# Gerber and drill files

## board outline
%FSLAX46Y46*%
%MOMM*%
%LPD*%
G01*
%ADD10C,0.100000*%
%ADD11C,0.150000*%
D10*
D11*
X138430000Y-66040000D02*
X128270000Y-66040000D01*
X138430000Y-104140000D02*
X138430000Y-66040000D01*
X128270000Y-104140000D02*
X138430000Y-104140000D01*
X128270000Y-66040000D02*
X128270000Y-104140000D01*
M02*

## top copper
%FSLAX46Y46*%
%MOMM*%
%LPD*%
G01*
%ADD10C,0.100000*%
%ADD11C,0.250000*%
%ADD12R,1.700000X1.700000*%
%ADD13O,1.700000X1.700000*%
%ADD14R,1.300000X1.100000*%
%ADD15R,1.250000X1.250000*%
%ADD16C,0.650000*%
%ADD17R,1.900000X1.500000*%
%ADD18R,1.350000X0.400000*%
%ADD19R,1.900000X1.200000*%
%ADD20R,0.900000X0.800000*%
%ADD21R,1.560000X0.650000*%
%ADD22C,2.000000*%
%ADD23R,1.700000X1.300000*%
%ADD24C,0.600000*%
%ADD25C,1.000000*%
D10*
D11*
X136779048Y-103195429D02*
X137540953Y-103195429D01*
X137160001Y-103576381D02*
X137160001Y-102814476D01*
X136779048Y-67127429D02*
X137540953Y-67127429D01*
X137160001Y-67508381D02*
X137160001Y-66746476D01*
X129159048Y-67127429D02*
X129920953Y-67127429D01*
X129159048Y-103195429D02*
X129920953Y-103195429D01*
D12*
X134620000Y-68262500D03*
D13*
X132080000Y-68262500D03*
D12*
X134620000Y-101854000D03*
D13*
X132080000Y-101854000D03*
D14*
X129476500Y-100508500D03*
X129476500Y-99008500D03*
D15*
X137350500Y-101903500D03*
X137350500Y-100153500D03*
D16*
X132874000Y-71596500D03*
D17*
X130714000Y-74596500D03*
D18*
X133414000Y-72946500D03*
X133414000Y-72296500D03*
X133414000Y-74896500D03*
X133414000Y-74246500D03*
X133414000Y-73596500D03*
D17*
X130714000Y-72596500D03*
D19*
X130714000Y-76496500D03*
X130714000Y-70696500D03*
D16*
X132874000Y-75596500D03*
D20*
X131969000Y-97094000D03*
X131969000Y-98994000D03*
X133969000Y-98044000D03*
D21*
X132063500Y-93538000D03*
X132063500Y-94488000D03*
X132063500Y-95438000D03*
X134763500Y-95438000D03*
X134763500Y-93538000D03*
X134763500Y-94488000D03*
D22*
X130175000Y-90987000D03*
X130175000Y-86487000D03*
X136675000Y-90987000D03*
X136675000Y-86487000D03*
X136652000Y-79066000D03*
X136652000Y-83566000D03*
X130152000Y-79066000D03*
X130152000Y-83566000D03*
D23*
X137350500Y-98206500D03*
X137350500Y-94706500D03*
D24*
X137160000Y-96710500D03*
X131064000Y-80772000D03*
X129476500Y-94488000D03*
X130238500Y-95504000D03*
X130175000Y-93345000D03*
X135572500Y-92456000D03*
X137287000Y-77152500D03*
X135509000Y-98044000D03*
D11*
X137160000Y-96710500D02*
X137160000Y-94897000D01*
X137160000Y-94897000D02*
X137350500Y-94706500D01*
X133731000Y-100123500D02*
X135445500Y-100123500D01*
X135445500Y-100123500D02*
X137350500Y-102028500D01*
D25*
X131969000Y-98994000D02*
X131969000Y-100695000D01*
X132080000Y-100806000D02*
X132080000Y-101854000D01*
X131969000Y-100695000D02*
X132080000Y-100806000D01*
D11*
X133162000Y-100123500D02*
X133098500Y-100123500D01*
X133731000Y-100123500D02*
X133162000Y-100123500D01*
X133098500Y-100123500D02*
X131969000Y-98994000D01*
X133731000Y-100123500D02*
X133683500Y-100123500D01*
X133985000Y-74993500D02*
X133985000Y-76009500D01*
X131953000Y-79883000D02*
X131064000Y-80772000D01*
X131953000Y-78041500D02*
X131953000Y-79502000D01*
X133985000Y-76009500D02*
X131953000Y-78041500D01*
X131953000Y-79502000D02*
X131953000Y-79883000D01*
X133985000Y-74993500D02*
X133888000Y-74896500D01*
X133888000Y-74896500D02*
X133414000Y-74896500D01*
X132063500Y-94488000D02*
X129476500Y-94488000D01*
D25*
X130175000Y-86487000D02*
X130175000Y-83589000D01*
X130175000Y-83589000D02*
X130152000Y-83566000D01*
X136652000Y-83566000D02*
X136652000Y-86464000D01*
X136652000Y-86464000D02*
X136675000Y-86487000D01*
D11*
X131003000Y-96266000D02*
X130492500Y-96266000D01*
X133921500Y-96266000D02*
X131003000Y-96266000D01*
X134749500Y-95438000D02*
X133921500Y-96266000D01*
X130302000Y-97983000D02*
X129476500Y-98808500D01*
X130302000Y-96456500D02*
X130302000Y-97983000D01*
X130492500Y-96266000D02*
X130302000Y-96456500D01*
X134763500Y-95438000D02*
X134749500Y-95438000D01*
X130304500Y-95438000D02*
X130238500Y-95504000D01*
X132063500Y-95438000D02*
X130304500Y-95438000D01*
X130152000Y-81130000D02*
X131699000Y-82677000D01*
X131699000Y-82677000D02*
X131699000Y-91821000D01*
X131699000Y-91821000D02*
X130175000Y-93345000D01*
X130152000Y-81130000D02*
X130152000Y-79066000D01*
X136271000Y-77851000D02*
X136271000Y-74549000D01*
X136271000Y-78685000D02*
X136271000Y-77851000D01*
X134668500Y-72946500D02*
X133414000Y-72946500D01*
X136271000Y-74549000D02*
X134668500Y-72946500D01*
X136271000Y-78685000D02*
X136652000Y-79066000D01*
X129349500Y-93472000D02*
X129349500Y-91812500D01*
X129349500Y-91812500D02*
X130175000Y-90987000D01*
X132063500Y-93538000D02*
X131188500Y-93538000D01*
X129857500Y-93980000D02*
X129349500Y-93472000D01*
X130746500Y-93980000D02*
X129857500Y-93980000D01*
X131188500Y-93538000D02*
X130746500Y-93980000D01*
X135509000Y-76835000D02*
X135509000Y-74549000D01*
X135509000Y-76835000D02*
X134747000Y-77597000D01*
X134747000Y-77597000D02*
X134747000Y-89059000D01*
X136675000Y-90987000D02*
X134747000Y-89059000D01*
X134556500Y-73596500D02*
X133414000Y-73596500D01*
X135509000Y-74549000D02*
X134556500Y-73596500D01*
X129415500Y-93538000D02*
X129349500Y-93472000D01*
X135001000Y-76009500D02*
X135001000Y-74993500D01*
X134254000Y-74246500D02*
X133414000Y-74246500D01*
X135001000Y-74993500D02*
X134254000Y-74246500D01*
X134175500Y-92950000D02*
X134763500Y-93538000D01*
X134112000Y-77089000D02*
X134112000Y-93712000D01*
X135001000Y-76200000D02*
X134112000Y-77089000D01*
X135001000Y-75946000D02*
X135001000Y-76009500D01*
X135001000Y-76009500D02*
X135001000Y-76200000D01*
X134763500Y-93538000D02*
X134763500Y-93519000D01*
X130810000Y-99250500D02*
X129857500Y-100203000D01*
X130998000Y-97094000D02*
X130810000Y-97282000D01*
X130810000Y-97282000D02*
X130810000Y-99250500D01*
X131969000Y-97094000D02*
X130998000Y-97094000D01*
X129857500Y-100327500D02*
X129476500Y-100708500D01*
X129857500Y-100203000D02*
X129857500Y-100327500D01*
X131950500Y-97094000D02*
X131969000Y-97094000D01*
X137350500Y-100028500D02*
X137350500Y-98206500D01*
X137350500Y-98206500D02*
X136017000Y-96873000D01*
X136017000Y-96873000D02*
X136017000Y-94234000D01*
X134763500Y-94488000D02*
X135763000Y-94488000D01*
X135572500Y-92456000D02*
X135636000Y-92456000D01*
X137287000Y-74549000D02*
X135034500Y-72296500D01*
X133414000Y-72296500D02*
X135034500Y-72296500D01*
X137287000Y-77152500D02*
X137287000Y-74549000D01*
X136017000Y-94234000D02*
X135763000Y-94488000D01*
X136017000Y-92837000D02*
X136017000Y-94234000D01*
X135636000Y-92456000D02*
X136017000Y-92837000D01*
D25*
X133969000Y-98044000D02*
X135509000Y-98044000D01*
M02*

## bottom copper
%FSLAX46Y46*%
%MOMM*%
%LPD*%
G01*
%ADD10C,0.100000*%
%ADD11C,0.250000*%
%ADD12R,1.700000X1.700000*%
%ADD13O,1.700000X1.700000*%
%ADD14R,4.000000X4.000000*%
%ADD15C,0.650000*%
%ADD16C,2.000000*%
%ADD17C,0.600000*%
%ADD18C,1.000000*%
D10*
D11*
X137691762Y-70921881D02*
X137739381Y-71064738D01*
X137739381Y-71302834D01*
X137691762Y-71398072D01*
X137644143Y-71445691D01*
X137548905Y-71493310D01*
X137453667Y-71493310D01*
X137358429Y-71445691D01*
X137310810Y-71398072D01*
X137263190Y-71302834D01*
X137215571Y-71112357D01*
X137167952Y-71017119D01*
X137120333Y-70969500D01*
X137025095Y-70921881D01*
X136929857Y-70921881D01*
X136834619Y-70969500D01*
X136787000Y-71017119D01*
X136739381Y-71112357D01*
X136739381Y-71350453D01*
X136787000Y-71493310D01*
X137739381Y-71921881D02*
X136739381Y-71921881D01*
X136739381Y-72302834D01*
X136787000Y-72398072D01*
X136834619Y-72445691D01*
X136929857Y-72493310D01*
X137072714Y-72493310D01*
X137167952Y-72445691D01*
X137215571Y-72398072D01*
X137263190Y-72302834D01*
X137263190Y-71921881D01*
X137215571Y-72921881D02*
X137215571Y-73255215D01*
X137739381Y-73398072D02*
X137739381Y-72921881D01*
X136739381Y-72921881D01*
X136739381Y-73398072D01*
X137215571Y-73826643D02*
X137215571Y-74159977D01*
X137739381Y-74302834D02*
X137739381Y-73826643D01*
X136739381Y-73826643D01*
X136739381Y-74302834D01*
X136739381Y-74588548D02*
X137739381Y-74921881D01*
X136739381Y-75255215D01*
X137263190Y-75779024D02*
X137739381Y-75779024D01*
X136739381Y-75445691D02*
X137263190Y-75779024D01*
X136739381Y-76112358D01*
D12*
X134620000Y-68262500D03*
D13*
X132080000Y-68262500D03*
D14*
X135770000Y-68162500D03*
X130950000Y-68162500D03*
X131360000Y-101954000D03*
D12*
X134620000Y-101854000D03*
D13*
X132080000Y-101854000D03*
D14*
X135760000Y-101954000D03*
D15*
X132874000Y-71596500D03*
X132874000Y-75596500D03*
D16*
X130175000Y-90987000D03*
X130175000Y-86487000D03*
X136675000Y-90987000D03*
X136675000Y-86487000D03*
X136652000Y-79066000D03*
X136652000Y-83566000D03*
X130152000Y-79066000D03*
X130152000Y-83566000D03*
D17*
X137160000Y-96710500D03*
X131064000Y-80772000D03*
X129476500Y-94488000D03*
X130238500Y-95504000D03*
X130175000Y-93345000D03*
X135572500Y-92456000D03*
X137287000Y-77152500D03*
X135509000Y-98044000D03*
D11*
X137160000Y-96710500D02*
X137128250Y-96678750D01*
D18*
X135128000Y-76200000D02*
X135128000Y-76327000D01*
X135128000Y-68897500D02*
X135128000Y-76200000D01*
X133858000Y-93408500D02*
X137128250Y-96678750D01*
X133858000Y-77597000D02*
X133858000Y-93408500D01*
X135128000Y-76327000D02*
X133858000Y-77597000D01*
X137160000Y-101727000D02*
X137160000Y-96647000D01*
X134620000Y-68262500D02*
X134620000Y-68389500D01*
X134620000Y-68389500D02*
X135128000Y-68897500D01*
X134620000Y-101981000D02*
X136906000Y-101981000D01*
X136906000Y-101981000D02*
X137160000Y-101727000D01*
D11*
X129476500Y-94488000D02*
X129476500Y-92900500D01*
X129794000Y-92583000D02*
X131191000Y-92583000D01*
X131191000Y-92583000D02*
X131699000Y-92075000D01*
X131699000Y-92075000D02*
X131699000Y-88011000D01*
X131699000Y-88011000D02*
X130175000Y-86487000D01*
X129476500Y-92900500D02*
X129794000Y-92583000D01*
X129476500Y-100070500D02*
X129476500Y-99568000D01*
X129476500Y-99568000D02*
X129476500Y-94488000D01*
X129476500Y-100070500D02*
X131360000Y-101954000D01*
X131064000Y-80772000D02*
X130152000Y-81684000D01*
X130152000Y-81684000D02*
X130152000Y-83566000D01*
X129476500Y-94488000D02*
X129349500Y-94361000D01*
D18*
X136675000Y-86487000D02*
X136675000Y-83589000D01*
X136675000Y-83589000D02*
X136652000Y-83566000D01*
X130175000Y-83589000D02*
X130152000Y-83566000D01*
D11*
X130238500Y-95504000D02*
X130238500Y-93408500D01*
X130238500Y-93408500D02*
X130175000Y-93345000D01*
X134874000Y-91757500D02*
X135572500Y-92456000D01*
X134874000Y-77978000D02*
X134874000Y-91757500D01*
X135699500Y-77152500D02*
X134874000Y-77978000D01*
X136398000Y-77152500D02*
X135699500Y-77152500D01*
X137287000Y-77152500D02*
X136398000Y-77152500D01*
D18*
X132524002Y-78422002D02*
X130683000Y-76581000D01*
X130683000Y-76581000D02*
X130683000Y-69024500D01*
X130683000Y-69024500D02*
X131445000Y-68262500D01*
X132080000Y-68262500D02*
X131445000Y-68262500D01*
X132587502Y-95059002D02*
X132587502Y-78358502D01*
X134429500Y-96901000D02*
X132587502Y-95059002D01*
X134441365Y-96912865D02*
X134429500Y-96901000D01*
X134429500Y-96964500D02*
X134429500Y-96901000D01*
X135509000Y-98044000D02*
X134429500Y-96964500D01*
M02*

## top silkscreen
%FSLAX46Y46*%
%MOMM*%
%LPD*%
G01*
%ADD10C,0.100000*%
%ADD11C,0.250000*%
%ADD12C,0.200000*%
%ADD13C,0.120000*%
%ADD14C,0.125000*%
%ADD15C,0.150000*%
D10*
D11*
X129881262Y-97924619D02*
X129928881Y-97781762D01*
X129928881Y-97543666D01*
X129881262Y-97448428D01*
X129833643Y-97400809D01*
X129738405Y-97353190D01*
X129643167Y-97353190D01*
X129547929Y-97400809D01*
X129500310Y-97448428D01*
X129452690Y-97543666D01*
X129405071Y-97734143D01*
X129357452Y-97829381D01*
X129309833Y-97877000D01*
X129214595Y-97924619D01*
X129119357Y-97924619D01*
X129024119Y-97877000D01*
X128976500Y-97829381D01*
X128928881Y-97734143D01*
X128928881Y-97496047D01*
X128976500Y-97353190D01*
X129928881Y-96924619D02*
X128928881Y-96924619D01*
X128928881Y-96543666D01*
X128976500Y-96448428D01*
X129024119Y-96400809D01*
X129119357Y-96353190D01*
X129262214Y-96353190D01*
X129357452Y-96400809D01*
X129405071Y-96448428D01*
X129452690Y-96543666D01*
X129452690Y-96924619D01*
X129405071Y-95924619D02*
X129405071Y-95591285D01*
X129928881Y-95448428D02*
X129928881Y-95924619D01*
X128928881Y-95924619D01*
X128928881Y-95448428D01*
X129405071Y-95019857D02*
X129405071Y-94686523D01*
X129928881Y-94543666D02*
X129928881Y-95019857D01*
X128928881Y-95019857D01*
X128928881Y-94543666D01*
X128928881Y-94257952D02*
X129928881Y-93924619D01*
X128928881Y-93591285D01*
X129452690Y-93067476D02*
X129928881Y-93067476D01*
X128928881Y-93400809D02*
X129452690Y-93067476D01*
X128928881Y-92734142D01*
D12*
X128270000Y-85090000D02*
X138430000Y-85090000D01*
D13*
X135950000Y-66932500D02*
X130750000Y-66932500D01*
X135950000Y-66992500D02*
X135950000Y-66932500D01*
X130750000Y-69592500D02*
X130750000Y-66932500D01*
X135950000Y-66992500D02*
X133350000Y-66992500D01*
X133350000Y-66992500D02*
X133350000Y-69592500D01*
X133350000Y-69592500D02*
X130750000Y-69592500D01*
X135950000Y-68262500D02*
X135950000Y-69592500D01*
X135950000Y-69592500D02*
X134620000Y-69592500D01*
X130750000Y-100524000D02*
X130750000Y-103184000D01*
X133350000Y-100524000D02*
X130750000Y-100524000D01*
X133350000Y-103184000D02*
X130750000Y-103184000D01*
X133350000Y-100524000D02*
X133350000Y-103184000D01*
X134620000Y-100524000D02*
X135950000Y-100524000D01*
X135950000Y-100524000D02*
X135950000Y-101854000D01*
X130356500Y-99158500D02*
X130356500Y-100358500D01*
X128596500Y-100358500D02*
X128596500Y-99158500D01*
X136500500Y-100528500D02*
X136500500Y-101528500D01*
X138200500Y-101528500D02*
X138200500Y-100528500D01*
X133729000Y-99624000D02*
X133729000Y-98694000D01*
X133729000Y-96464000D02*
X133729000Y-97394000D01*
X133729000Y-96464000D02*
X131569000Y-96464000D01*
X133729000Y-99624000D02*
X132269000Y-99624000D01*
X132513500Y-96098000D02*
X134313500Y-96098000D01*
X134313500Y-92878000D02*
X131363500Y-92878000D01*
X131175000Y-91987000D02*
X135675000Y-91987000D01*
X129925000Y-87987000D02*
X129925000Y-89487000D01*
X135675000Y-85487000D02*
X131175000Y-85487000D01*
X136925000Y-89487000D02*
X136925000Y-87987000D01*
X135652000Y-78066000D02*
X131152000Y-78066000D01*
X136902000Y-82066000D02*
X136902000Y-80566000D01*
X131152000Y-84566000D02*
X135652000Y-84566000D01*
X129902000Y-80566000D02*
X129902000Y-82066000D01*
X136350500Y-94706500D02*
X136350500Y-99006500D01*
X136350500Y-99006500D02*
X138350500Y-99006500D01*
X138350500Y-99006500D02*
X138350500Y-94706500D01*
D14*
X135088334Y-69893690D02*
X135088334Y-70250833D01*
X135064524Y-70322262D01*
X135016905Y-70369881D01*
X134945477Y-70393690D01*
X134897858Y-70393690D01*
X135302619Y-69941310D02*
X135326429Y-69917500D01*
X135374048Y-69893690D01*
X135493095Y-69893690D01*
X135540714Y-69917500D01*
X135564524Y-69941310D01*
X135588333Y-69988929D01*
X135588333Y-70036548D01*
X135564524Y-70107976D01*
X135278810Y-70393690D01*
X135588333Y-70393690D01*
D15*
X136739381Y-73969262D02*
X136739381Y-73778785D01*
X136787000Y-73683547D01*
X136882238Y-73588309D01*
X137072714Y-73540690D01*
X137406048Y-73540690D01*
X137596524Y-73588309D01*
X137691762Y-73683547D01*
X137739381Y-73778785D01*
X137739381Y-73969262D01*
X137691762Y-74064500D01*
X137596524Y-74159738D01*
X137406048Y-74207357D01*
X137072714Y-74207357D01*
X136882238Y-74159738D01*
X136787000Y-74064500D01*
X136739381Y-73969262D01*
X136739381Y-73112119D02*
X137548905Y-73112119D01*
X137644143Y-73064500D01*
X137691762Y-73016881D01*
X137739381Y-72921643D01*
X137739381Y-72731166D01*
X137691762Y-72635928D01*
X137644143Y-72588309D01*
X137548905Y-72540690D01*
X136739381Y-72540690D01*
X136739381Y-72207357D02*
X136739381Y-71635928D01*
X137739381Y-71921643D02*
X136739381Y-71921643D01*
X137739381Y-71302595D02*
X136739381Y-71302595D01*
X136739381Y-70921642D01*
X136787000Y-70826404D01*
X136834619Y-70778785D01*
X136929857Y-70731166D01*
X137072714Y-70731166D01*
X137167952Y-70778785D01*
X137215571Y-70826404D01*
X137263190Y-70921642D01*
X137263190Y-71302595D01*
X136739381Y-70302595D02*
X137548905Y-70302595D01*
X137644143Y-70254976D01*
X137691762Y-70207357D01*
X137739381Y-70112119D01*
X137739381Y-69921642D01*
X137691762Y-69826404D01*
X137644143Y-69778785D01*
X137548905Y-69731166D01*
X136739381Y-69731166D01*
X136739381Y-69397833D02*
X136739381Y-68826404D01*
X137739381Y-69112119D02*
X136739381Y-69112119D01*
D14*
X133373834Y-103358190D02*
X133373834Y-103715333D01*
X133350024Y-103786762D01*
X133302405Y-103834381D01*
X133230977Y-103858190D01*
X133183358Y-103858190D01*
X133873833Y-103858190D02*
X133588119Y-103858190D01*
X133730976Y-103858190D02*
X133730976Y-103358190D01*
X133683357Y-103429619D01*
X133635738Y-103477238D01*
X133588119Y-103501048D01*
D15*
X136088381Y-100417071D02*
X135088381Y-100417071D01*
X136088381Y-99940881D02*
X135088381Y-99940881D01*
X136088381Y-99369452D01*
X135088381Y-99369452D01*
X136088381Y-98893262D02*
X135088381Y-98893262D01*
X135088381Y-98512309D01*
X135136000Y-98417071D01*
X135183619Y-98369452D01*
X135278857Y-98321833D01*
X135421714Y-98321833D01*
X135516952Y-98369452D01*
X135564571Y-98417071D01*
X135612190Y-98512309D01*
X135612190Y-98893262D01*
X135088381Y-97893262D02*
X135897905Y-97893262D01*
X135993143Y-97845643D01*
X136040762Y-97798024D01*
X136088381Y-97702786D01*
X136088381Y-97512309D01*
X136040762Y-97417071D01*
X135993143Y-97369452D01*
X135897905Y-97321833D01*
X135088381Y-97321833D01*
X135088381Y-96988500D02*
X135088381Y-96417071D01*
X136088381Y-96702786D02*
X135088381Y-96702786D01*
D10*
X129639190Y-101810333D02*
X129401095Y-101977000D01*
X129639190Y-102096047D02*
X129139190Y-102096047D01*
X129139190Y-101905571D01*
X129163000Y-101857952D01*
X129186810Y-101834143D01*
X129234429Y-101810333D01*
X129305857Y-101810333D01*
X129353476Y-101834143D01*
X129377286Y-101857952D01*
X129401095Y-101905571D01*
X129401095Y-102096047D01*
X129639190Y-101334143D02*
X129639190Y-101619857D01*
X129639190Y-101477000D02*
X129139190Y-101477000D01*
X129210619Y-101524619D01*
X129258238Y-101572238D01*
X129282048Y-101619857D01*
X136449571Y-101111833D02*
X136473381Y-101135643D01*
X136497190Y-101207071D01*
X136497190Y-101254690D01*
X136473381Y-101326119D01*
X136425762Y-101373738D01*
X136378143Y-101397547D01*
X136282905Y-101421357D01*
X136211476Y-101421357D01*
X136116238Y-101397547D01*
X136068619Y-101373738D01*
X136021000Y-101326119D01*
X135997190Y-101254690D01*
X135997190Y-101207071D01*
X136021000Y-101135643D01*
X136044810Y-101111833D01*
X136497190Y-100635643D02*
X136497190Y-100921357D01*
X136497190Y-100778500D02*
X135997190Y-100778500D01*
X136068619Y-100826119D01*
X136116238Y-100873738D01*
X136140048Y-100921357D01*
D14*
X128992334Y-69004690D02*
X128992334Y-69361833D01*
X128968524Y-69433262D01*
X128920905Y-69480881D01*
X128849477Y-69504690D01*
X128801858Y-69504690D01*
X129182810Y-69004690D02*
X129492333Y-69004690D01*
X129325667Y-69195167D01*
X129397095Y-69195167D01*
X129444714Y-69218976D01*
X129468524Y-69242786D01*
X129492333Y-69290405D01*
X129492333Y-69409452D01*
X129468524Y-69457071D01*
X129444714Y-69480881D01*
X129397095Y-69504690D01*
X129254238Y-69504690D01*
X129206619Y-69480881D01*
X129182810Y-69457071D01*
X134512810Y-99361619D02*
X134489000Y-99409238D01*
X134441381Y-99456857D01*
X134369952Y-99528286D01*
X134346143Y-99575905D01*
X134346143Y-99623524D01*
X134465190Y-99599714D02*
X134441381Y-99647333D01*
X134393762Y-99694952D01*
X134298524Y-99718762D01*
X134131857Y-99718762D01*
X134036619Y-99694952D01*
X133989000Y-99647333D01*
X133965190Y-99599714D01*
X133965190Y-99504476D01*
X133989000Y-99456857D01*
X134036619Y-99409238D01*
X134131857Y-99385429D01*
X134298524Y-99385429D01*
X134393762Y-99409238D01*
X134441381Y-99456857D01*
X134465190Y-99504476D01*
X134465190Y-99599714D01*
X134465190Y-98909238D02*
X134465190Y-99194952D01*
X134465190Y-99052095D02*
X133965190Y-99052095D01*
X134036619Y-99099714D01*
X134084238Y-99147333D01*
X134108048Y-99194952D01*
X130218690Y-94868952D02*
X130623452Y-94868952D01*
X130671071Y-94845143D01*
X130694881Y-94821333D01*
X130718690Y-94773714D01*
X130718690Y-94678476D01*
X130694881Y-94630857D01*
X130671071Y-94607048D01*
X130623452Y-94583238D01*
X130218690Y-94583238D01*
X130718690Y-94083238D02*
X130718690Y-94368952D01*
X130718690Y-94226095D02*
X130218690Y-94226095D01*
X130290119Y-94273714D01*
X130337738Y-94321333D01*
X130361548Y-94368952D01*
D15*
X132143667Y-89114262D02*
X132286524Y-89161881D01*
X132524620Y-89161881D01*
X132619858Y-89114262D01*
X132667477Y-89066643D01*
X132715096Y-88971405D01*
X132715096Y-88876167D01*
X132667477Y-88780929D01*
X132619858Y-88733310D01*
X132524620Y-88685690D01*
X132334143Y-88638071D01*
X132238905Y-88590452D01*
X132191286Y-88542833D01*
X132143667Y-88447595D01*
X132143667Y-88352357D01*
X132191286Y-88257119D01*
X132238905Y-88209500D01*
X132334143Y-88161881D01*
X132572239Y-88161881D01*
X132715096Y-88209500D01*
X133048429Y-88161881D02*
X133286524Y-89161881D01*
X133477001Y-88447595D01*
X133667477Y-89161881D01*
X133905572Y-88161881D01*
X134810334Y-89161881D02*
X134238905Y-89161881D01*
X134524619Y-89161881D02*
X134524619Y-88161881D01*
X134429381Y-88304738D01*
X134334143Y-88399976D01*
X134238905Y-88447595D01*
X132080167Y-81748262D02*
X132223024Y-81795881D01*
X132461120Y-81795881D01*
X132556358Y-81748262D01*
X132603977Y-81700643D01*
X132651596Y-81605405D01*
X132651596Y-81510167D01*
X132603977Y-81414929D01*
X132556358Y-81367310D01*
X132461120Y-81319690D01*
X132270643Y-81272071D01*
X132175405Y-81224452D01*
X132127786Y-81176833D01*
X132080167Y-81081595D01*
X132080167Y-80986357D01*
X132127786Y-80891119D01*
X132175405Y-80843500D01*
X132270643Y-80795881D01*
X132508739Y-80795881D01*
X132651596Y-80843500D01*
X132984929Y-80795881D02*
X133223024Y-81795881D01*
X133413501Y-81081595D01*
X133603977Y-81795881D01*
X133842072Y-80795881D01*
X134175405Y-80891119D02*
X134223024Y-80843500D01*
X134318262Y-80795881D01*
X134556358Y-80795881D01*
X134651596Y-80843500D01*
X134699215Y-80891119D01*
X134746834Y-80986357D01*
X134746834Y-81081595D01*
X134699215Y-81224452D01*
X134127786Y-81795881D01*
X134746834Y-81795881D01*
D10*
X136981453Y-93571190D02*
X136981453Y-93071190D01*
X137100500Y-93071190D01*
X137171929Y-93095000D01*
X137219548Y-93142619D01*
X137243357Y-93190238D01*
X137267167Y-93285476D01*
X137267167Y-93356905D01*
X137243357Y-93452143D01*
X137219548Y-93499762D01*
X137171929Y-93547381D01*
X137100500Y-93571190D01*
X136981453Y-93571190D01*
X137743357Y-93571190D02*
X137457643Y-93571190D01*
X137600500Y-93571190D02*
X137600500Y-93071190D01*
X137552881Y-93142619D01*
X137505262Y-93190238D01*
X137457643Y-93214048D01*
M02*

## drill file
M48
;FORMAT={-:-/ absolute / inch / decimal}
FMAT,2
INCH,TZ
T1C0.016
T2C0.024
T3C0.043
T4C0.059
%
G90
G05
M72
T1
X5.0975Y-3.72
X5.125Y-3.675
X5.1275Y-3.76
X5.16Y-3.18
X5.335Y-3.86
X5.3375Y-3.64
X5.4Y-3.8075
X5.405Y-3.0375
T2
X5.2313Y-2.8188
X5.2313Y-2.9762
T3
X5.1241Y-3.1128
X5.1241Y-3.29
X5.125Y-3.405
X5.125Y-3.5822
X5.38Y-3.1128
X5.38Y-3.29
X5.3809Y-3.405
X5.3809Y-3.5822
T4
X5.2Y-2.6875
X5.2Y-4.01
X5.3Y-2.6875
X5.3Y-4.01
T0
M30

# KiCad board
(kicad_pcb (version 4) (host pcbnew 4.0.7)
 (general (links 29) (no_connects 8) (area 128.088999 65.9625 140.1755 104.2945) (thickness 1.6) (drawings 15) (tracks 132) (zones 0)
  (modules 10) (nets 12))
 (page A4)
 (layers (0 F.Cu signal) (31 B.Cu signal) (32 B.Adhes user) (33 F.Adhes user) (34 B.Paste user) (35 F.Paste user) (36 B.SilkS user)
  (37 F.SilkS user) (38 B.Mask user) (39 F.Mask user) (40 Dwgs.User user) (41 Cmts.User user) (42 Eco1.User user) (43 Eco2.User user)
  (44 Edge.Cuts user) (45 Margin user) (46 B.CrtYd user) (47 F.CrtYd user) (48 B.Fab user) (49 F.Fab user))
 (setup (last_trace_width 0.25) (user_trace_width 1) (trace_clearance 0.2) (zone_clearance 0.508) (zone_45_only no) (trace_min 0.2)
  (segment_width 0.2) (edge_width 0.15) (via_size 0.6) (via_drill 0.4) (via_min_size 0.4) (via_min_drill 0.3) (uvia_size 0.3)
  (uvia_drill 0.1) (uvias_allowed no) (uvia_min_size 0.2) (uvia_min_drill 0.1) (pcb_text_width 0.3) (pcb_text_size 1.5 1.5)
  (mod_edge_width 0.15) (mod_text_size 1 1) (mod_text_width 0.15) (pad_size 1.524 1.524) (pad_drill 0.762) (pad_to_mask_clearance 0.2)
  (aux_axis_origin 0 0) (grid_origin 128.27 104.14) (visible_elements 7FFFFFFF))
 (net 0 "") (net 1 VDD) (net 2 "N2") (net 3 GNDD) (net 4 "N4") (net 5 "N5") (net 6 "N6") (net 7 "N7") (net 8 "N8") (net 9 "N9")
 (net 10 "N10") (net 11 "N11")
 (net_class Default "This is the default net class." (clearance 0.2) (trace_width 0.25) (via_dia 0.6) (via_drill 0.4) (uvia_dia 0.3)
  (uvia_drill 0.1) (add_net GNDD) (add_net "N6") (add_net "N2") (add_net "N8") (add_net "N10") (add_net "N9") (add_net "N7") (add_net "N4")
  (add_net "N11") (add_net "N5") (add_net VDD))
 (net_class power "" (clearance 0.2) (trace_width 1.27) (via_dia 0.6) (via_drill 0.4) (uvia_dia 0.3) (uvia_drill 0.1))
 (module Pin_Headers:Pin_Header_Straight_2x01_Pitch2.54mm (layer F.Cu) (at 134.62 68.2625 180)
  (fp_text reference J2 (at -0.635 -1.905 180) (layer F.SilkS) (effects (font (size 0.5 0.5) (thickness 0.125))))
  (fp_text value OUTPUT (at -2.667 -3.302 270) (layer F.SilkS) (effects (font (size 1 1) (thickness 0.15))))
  (fp_line (start -1.33 1.33) (end 3.87 1.33) (layer F.SilkS) (width 0.12))
  (fp_line (start -1.33 1.27) (end -1.33 1.33) (layer F.SilkS) (width 0.12))
  (fp_line (start 3.87 -1.33) (end 3.87 1.33) (layer F.SilkS) (width 0.12))
  (fp_line (start -1.33 1.27) (end 1.27 1.27) (layer F.SilkS) (width 0.12))
  (fp_line (start 1.27 1.27) (end 1.27 -1.33) (layer F.SilkS) (width 0.12))
  (fp_line (start 1.27 -1.33) (end 3.87 -1.33) (layer F.SilkS) (width 0.12))
  (fp_line (start -1.33 0) (end -1.33 -1.33) (layer F.SilkS) (width 0.12))
  (fp_line (start -1.33 -1.33) (end 0 -1.33) (layer F.SilkS) (width 0.12))
  (pad 1 thru_hole rect (at 0 0 180) (size 1.7 1.7) (drill 1.5) (layers *.Cu *.Mask) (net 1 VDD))
  (pad 2 thru_hole oval (at 2.54 0 180) (size 1.7 1.7) (drill 1.5) (layers *.Cu *.Mask) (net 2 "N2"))
  (pad 1 smd rect (at -1.15 0.1 180) (size 4 4) (layers B.Cu B.Paste B.Mask) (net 1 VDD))
  (pad 2 smd rect (at 3.67 0.1 180) (size 4 4) (layers B.Cu B.Paste B.Mask) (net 2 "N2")))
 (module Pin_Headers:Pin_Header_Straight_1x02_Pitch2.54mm (layer F.Cu) (at 134.62 101.854 270)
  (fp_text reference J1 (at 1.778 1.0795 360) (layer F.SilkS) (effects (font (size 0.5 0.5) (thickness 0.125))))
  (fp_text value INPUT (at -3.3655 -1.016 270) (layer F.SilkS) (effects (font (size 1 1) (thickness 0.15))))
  (fp_line (start -1.33 3.87) (end 1.33 3.87) (layer F.SilkS) (width 0.12))
  (fp_line (start -1.33 1.27) (end -1.33 3.87) (layer F.SilkS) (width 0.12))
  (fp_line (start 1.33 1.27) (end 1.33 3.87) (layer F.SilkS) (width 0.12))
  (fp_line (start -1.33 1.27) (end 1.33 1.27) (layer F.SilkS) (width 0.12))
  (fp_line (start -1.33 0) (end -1.33 -1.33) (layer F.SilkS) (width 0.12))
  (fp_line (start -1.33 -1.33) (end 0 -1.33) (layer F.SilkS) (width 0.12))
  (pad 2 smd rect (at 0.1 3.26 270) (size 4 4) (layers B.Cu B.Paste B.Mask) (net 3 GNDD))
  (pad 1 thru_hole rect (at 0 0 270) (size 1.7 1.7) (drill 1.5) (layers *.Cu *.Mask) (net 1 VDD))
  (pad 2 thru_hole oval (at 0 2.54 270) (size 1.7 1.7) (drill 1.5) (layers *.Cu *.Mask) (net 3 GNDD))
  (pad 1 smd rect (at 0.1 -1.14 270) (size 4 4) (layers B.Cu B.Paste B.Mask) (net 1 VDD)))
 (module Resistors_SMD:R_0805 (layer F.Cu) (at 129.4765 99.7585 90)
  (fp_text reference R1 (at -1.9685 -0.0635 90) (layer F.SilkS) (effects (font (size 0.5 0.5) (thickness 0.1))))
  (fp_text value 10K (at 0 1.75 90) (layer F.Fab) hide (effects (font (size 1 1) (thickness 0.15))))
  (fp_line (start 0.6 0.88) (end -0.6 0.88) (layer F.SilkS) (width 0.12))
  (fp_line (start -0.6 -0.88) (end 0.6 -0.88) (layer F.SilkS) (width 0.12))
  (pad 1 smd rect (at -0.75 0 90) (size 1.1 1.3) (layers F.Cu F.Paste F.Mask) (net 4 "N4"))
  (pad 2 smd rect (at 0.75 0 90) (size 1.1 1.3) (layers F.Cu F.Paste F.Mask) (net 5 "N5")))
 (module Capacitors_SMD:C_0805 (layer F.Cu) (at 137.3505 101.0285 90)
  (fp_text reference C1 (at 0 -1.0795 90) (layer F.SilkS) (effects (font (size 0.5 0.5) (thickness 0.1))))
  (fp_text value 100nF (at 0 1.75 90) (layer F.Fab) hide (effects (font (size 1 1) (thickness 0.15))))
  (fp_line (start 0.5 -0.85) (end -0.5 -0.85) (layer F.SilkS) (width 0.12))
  (fp_line (start -0.5 0.85) (end 0.5 0.85) (layer F.SilkS) (width 0.12))
  (pad 1 smd rect (at -0.875 0 90) (size 1.25 1.25) (layers F.Cu F.Paste F.Mask) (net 3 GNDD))
  (pad 2 smd rect (at 0.875 0 90) (size 1.25 1.25) (layers F.Cu F.Paste F.Mask) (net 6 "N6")))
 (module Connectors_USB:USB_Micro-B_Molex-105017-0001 (layer F.Cu) (at 131.064 73.5965 270)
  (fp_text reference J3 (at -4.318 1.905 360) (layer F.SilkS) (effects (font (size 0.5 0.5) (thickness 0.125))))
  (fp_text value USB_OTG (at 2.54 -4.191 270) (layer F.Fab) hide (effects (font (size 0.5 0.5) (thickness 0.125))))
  (pad 6 thru_hole circle (at -2 -1.81 270) (size 0.65 0.65) (drill 0.6) (layers *.Cu *.Mask) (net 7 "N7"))
  (pad 6 smd rect (at 1 0.35 270) (size 1.5 1.9) (layers F.Cu F.Paste F.Mask) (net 7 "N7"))
  (pad 2 smd rect (at -0.65 -2.35 270) (size 0.4 1.35) (layers F.Cu F.Paste F.Mask) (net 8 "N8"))
  (pad 1 smd rect (at -1.3 -2.35 270) (size 0.4 1.35) (layers F.Cu F.Paste F.Mask) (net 6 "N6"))
  (pad 5 smd rect (at 1.3 -2.35 270) (size 0.4 1.35) (layers F.Cu F.Paste F.Mask) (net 3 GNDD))
  (pad 4 smd rect (at 0.65 -2.35 270) (size 0.4 1.35) (layers F.Cu F.Paste F.Mask) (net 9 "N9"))
  (pad 3 smd rect (at 0 -2.35 270) (size 0.4 1.35) (layers F.Cu F.Paste F.Mask) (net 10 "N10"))
  (pad 6 smd rect (at -1 0.35 270) (size 1.5 1.9) (layers F.Cu F.Paste F.Mask) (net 7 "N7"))
  (pad 6 smd rect (at 2.9 0.35 270) (size 1.2 1.9) (layers F.Cu F.Mask) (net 7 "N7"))
  (pad 6 smd rect (at -2.9 0.35 270) (size 1.2 1.9) (layers F.Cu F.Mask) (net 7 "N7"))
  (pad 6 thru_hole circle (at 2 -1.81 270) (size 0.65 0.65) (drill 0.6) (layers *.Cu *.Mask) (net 7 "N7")))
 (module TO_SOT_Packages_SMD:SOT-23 (layer F.Cu) (at 132.969 98.044)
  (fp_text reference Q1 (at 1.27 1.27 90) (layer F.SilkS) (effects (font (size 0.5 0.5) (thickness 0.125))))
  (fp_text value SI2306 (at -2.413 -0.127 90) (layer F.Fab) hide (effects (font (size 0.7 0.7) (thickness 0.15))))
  (fp_line (start 0.76 1.58) (end 0.76 0.65) (layer F.SilkS) (width 0.12))
  (fp_line (start 0.76 -1.58) (end 0.76 -0.65) (layer F.SilkS) (width 0.12))
  (fp_line (start 0.76 -1.58) (end -1.4 -1.58) (layer F.SilkS) (width 0.12))
  (fp_line (start 0.76 1.58) (end -0.7 1.58) (layer F.SilkS) (width 0.12))
  (pad 1 smd rect (at -1 -0.95) (size 0.9 0.8) (layers F.Cu F.Paste F.Mask) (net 4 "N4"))
  (pad 2 smd rect (at -1 0.95) (size 0.9 0.8) (layers F.Cu F.Paste F.Mask) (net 3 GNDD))
  (pad 3 smd rect (at 1 0) (size 0.9 0.8) (layers F.Cu F.Paste F.Mask) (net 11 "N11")))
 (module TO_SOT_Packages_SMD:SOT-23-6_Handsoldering (layer F.Cu) (at 133.4135 94.488)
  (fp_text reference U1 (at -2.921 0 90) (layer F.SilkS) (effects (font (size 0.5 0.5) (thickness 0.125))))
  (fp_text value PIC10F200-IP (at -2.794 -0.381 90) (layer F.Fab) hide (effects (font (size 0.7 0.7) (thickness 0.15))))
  (fp_line (start -0.9 1.61) (end 0.9 1.61) (layer F.SilkS) (width 0.12))
  (fp_line (start 0.9 -1.61) (end -2.05 -1.61) (layer F.SilkS) (width 0.12))
  (pad 1 smd rect (at -1.35 -0.95) (size 1.56 0.65) (layers F.Cu F.Paste F.Mask) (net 10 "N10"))
  (pad 2 smd rect (at -1.35 0) (size 1.56 0.65) (layers F.Cu F.Paste F.Mask) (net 3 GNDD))
  (pad 3 smd rect (at -1.35 0.95) (size 1.56 0.65) (layers F.Cu F.Paste F.Mask) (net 8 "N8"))
  (pad 4 smd rect (at 1.35 0.95) (size 1.56 0.65) (layers F.Cu F.Paste F.Mask) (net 5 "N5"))
  (pad 6 smd rect (at 1.35 -0.95) (size 1.56 0.65) (layers F.Cu F.Paste F.Mask) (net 9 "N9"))
  (pad 5 smd rect (at 1.35 0) (size 1.56 0.65) (layers F.Cu F.Paste F.Mask) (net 6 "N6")))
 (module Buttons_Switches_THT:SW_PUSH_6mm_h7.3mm (layer F.Cu) (at 130.175 86.487)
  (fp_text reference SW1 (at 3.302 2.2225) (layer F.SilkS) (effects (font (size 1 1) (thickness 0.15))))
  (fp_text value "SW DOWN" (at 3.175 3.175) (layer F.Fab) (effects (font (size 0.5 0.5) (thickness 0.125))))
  (fp_line (start 1 5.5) (end 5.5 5.5) (layer F.SilkS) (width 0.12))
  (fp_line (start -0.25 1.5) (end -0.25 3) (layer F.SilkS) (width 0.12))
  (fp_line (start 5.5 -1) (end 1 -1) (layer F.SilkS) (width 0.12))
  (fp_line (start 6.75 3) (end 6.75 1.5) (layer F.SilkS) (width 0.12))
  (pad 2 thru_hole circle (at 0 4.5 90) (size 2 2) (drill 1.1) (layers *.Cu *.Mask) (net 10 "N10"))
  (pad 1 thru_hole circle (at 0 0 90) (size 2 2) (drill 1.1) (layers *.Cu *.Mask) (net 3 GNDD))
  (pad 2 thru_hole circle (at 6.5 4.5 90) (size 2 2) (drill 1.1) (layers *.Cu *.Mask) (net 10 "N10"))
  (pad 1 thru_hole circle (at 6.5 0 90) (size 2 2) (drill 1.1) (layers *.Cu *.Mask) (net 3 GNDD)))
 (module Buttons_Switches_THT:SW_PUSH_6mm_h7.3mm (layer F.Cu) (at 136.652 83.566 180)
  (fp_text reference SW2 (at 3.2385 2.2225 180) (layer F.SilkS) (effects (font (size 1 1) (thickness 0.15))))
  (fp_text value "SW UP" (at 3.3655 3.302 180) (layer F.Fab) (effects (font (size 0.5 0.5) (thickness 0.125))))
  (fp_line (start 1 5.5) (end 5.5 5.5) (layer F.SilkS) (width 0.12))
  (fp_line (start -0.25 1.5) (end -0.25 3) (layer F.SilkS) (width 0.12))
  (fp_line (start 5.5 -1) (end 1 -1) (layer F.SilkS) (width 0.12))
  (fp_line (start 6.75 3) (end 6.75 1.5) (layer F.SilkS) (width 0.12))
  (pad 2 thru_hole circle (at 0 4.5 270) (size 2 2) (drill 1.1) (layers *.Cu *.Mask) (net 8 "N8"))
  (pad 1 thru_hole circle (at 0 0 270) (size 2 2) (drill 1.1) (layers *.Cu *.Mask) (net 3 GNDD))
  (pad 2 thru_hole circle (at 6.5 4.5 270) (size 2 2) (drill 1.1) (layers *.Cu *.Mask) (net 8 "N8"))
  (pad 1 thru_hole circle (at 6.5 0 270) (size 2 2) (drill 1.1) (layers *.Cu *.Mask) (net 3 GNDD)))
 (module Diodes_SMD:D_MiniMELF (layer F.Cu) (at 137.3505 96.4565 90)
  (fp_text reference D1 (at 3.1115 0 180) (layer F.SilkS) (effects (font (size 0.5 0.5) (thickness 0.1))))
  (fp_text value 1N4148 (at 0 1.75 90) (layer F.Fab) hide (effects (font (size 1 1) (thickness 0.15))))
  (fp_line (start 1.75 -1) (end -2.55 -1) (layer F.SilkS) (width 0.12))
  (fp_line (start -2.55 -1) (end -2.55 1) (layer F.SilkS) (width 0.12))
  (fp_line (start -2.55 1) (end 1.75 1) (layer F.SilkS) (width 0.12))
  (pad 1 smd rect (at -1.75 0 90) (size 1.3 1.7) (layers F.Cu F.Paste F.Mask) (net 6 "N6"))
  (pad 2 smd rect (at 1.75 0 90) (size 1.3 1.7) (layers F.Cu F.Paste F.Mask) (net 1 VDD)))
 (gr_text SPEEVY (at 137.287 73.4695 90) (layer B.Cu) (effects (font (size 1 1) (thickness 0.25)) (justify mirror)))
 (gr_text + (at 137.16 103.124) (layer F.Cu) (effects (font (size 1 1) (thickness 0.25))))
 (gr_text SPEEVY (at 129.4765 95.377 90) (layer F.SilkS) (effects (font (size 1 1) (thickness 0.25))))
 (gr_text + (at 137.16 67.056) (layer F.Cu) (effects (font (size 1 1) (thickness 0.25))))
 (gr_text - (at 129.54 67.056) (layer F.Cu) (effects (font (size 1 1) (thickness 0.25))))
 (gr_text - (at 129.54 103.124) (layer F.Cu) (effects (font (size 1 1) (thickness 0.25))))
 (gr_line (start 128.27 85.09) (end 138.43 85.09) (angle 90) (layer F.SilkS) (width 0.2))
 (gr_line (start 138.43 66.04) (end 128.27 66.04) (angle 90) (layer Edge.Cuts) (width 0.15))
 (gr_line (start 138.43 104.14) (end 138.43 66.04) (angle 90) (layer Edge.Cuts) (width 0.15))
 (gr_line (start 128.27 104.14) (end 138.43 104.14) (angle 90) (layer Edge.Cuts) (width 0.15))
 (gr_line (start 128.27 66.04) (end 128.27 104.14) (angle 90) (layer Edge.Cuts) (width 0.15))
 (segment (start 137.16 96.7105) (end 137.16 94.897) (width 0.25) (layer F.Cu) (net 1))
 (segment (start 137.16 94.897) (end 137.3505 94.7065) (width 0.25) (layer F.Cu) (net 1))
 (segment (start 137.16 96.7105) (end 137.12825 96.67875) (width 0.25) (layer B.Cu) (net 1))
 (via (at 137.16 96.7105) (size 0.6) (drill 0.4) (layers F.Cu B.Cu) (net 1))
 (segment (start 135.128 76.2) (end 135.128 76.327) (width 1) (layer B.Cu) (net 1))
 (segment (start 135.128 68.8975) (end 135.128 76.2) (width 1) (layer B.Cu) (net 1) (status 10))
 (segment (start 133.858 93.4085) (end 137.12825 96.67875) (width 1) (layer B.Cu) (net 1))
 (segment (start 133.858 77.597) (end 133.858 93.4085) (width 1) (layer B.Cu) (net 1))
 (segment (start 135.128 76.327) (end 133.858 77.597) (width 1) (layer B.Cu) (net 1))
 (segment (start 137.16 101.727) (end 137.16 96.647) (width 1) (layer B.Cu) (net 1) (status 10))
 (segment (start 134.62 68.2625) (end 134.62 68.3895) (width 1) (layer B.Cu) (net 1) (status 30))
 (segment (start 134.62 68.3895) (end 135.128 68.8975) (width 1) (layer B.Cu) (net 1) (status 30))
 (segment (start 134.62 101.981) (end 136.906 101.981) (width 1) (layer B.Cu) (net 1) (status 30))
 (segment (start 136.906 101.981) (end 137.16 101.727) (width 1) (layer B.Cu) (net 1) (status 30))
 (segment (start 133.731 100.1235) (end 135.4455 100.1235) (width 0.25) (layer F.Cu) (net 3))
 (segment (start 135.4455 100.1235) (end 137.3505 102.0285) (width 0.25) (layer F.Cu) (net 3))
 (segment (start 131.969 98.994) (end 131.969 100.695) (width 1) (layer F.Cu) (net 3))
 (segment (start 132.08 100.806) (end 132.08 101.854) (width 1) (layer F.Cu) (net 3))
 (segment (start 131.969 100.695) (end 132.08 100.806) (width 1) (layer F.Cu) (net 3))
 (segment (start 133.162 100.1235) (end 133.0985 100.1235) (width 0.25) (layer F.Cu) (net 3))
 (segment (start 133.731 100.1235) (end 133.162 100.1235) (width 0.25) (layer F.Cu) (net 3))
 (segment (start 133.0985 100.1235) (end 131.969 98.994) (width 0.25) (layer F.Cu) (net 3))
 (segment (start 129.4765 94.488) (end 129.4765 92.9005) (width 0.25) (layer B.Cu) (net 3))
 (segment (start 129.794 92.583) (end 131.191 92.583) (width 0.25) (layer B.Cu) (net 3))
 (segment (start 131.191 92.583) (end 131.699 92.075) (width 0.25) (layer B.Cu) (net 3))
 (segment (start 131.699 92.075) (end 131.699 88.011) (width 0.25) (layer B.Cu) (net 3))
 (segment (start 131.699 88.011) (end 130.175 86.487) (width 0.25) (layer B.Cu) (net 3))
 (segment (start 129.4765 92.9005) (end 129.794 92.583) (width 0.25) (layer B.Cu) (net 3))
 (segment (start 129.4765 100.0705) (end 129.4765 99.568) (width 0.25) (layer B.Cu) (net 3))
 (segment (start 129.4765 99.568) (end 129.4765 94.488) (width 0.25) (layer B.Cu) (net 3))
 (segment (start 129.4765 100.0705) (end 131.36 101.954) (width 0.25) (layer B.Cu) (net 3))
 (segment (start 133.731 100.1235) (end 133.6835 100.1235) (width 0.25) (layer F.Cu) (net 3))
 (segment (start 133.985 74.9935) (end 133.985 76.0095) (width 0.25) (layer F.Cu) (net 3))
 (segment (start 131.953 79.883) (end 131.064 80.772) (width 0.25) (layer F.Cu) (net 3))
 (via (at 131.064 80.772) (size 0.6) (drill 0.4) (layers F.Cu B.Cu) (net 3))
 (segment (start 131.064 80.772) (end 130.152 81.684) (width 0.25) (layer B.Cu) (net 3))
 (segment (start 130.152 81.684) (end 130.152 83.566) (width 0.25) (layer B.Cu) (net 3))
 (segment (start 131.953 78.0415) (end 131.953 79.502) (width 0.25) (layer F.Cu) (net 3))
 (segment (start 133.985 76.0095) (end 131.953 78.0415) (width 0.25) (layer F.Cu) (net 3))
 (segment (start 131.953 79.502) (end 131.953 79.883) (width 0.25) (layer F.Cu) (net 3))
 (segment (start 133.985 74.9935) (end 133.888 74.8965) (width 0.25) (layer F.Cu) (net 3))
 (segment (start 133.888 74.8965) (end 133.414 74.8965) (width 0.25) (layer F.Cu) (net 3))
 (segment (start 132.0635 94.488) (end 129.4765 94.488) (width 0.25) (layer F.Cu) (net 3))
 (via (at 129.4765 94.488) (size 0.6) (drill 0.4) (layers F.Cu B.Cu) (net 3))
 (segment (start 129.4765 94.488) (end 129.3495 94.361) (width 0.25) (layer B.Cu) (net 3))
 (segment (start 130.175 86.487) (end 130.175 83.589) (width 1) (layer F.Cu) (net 3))
 (segment (start 130.175 83.589) (end 130.152 83.566) (width 1) (layer F.Cu) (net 3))
 (segment (start 136.652 83.566) (end 136.652 86.464) (width 1) (layer F.Cu) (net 3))
 (segment (start 136.652 86.464) (end 136.675 86.487) (width 1) (layer F.Cu) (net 3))
 (segment (start 136.675 86.487) (end 136.675 83.589) (width 1) (layer B.Cu) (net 3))
 (segment (start 136.675 83.589) (end 136.652 83.566) (width 1) (layer B.Cu) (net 3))
 (segment (start 130.175 83.589) (end 130.152 83.566) (width 1) (layer B.Cu) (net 3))
 (segment (start 131.003 96.266) (end 130.4925 96.266) (width 0.25) (layer F.Cu) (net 5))
 (segment (start 133.9215 96.266) (end 131.003 96.266) (width 0.25) (layer F.Cu) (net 5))
 (segment (start 134.7495 95.438) (end 133.9215 96.266) (width 0.25) (layer F.Cu) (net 5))
 (segment (start 130.302 97.983) (end 129.4765 98.8085) (width 0.25) (layer F.Cu) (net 5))
 (segment (start 130.302 96.4565) (end 130.302 97.983) (width 0.25) (layer F.Cu) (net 5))
 (segment (start 130.4925 96.266) (end 130.302 96.4565) (width 0.25) (layer F.Cu) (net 5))
 (segment (start 134.7635 95.438) (end 134.7495 95.438) (width 0.25) (layer F.Cu) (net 5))
 (segment (start 130.2385 95.504) (end 130.2385 93.4085) (width 0.25) (layer B.Cu) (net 8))
 (segment (start 130.3045 95.438) (end 130.2385 95.504) (width 0.25) (layer F.Cu) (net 8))
 (via (at 130.2385 95.504) (size 0.6) (drill 0.4) (layers F.Cu B.Cu) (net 8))
 (via (at 130.175 93.345) (size 0.6) (drill 0.4) (layers F.Cu B.Cu) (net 8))
 (segment (start 132.0635 95.438) (end 130.3045 95.438) (width 0.25) (layer F.Cu) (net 8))
 (segment (start 130.152 81.13) (end 131.699 82.677) (width 0.25) (layer F.Cu) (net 8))
 (segment (start 131.699 82.677) (end 131.699 91.821) (width 0.25) (layer F.Cu) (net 8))
 (segment (start 131.699 91.821) (end 130.175 93.345) (width 0.25) (layer F.Cu) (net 8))
 (segment (start 130.152 81.13) (end 130.152 79.066) (width 0.25) (layer F.Cu) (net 8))
 (segment (start 130.2385 93.4085) (end 130.175 93.345) (width 0.25) (layer B.Cu) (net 8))
 (segment (start 136.271 77.851) (end 136.271 74.549) (width 0.25) (layer F.Cu) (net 8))
 (segment (start 136.271 78.685) (end 136.271 77.851) (width 0.25) (layer F.Cu) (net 8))
 (segment (start 134.6685 72.9465) (end 133.414 72.9465) (width 0.25) (layer F.Cu) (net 8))
 (segment (start 136.271 74.549) (end 134.6685 72.9465) (width 0.25) (layer F.Cu) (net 8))
 (segment (start 136.271 78.685) (end 136.652 79.066) (width 0.25) (layer F.Cu) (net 8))
 (segment (start 129.3495 93.472) (end 129.3495 91.8125) (width 0.25) (layer F.Cu) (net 10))
 (segment (start 129.3495 91.8125) (end 130.175 90.987) (width 0.25) (layer F.Cu) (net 10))
 (segment (start 132.0635 93.538) (end 131.1885 93.538) (width 0.25) (layer F.Cu) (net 10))
 (segment (start 129.8575 93.98) (end 129.3495 93.472) (width 0.25) (layer F.Cu) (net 10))
 (segment (start 130.7465 93.98) (end 129.8575 93.98) (width 0.25) (layer F.Cu) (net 10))
 (segment (start 131.1885 93.538) (end 130.7465 93.98) (width 0.25) (layer F.Cu) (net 10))
 (segment (start 135.509 76.835) (end 135.509 74.549) (width 0.25) (layer F.Cu) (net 10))
 (segment (start 135.509 76.835) (end 134.747 77.597) (width 0.25) (layer F.Cu) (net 10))
 (segment (start 134.747 77.597) (end 134.747 89.059) (width 0.25) (layer F.Cu) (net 10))
 (segment (start 136.675 90.987) (end 134.747 89.059) (width 0.25) (layer F.Cu) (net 10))
 (segment (start 134.5565 73.5965) (end 133.414 73.5965) (width 0.25) (layer F.Cu) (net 10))
 (segment (start 135.509 74.549) (end 134.5565 73.5965) (width 0.25) (layer F.Cu) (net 10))
 (segment (start 129.4155 93.538) (end 129.3495 93.472) (width 0.25) (layer F.Cu) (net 10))
 (segment (start 135.001 76.0095) (end 135.001 74.9935) (width 0.25) (layer F.Cu) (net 9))
 (segment (start 134.254 74.2465) (end 133.414 74.2465) (width 0.25) (layer F.Cu) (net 9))
 (segment (start 135.001 74.9935) (end 134.254 74.2465) (width 0.25) (layer F.Cu) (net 9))
 (segment (start 134.1755 92.95) (end 134.7635 93.538) (width 0.25) (layer F.Cu) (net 9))
 (segment (start 134.112 77.089) (end 134.112 93.712) (width 0.25) (layer F.Cu) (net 9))
 (segment (start 135.001 76.2) (end 134.112 77.089) (width 0.25) (layer F.Cu) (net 9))
 (segment (start 135.001 75.946) (end 135.001 76.0095) (width 0.25) (layer F.Cu) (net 9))
 (segment (start 135.001 76.0095) (end 135.001 76.2) (width 0.25) (layer F.Cu) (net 9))
 (segment (start 134.7635 93.538) (end 134.7635 93.519) (width 0.25) (layer F.Cu) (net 9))
 (segment (start 130.81 99.2505) (end 129.8575 100.203) (width 0.25) (layer F.Cu) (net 4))
 (segment (start 130.998 97.094) (end 130.81 97.282) (width 0.25) (layer F.Cu) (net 4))
 (segment (start 130.81 97.282) (end 130.81 99.2505) (width 0.25) (layer F.Cu) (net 4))
 (segment (start 131.969 97.094) (end 130.998 97.094) (width 0.25) (layer F.Cu) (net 4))
 (segment (start 129.8575 100.3275) (end 129.4765 100.7085) (width 0.25) (layer F.Cu) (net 4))
 (segment (start 129.8575 100.203) (end 129.8575 100.3275) (width 0.25) (layer F.Cu) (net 4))
 (segment (start 131.9505 97.094) (end 131.969 97.094) (width 0.25) (layer F.Cu) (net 4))
 (segment (start 137.3505 100.0285) (end 137.3505 98.2065) (width 0.25) (layer F.Cu) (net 6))
 (segment (start 137.3505 98.2065) (end 136.017 96.873) (width 0.25) (layer F.Cu) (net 6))
 (segment (start 136.017 96.873) (end 136.017 94.234) (width 0.25) (layer F.Cu) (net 6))
 (segment (start 134.7635 94.488) (end 135.763 94.488) (width 0.25) (layer F.Cu) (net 6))
 (segment (start 135.5725 92.456) (end 135.636 92.456) (width 0.25) (layer F.Cu) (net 6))
 (segment (start 137.287 74.549) (end 135.0345 72.2965) (width 0.25) (layer F.Cu) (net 6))
 (segment (start 133.414 72.2965) (end 135.0345 72.2965) (width 0.25) (layer F.Cu) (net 6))
 (via (at 135.5725 92.456) (size 0.6) (drill 0.4) (layers F.Cu B.Cu) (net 6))
 (segment (start 134.874 91.7575) (end 135.5725 92.456) (width 0.25) (layer B.Cu) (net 6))
 (segment (start 134.874 77.978) (end 134.874 91.7575) (width 0.25) (layer B.Cu) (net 6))
 (segment (start 135.6995 77.1525) (end 134.874 77.978) (width 0.25) (layer B.Cu) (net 6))
 (segment (start 136.398 77.1525) (end 135.6995 77.1525) (width 0.25) (layer B.Cu) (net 6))
 (segment (start 137.287 77.1525) (end 136.398 77.1525) (width 0.25) (layer B.Cu) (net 6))
 (via (at 137.287 77.1525) (size 0.6) (drill 0.4) (layers F.Cu B.Cu) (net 6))
 (segment (start 137.287 77.1525) (end 137.287 74.549) (width 0.25) (layer F.Cu) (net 6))
 (segment (start 136.017 94.234) (end 135.763 94.488) (width 0.25) (layer F.Cu) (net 6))
 (segment (start 136.017 92.837) (end 136.017 94.234) (width 0.25) (layer F.Cu) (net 6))
 (segment (start 135.636 92.456) (end 136.017 92.837) (width 0.25) (layer F.Cu) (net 6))
 (segment (start 132.524002 78.422002) (end 130.683 76.581) (width 1) (layer B.Cu) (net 11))
 (segment (start 130.683 76.581) (end 130.683 69.0245) (width 1) (layer B.Cu) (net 11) (status 20))
 (segment (start 130.683 69.0245) (end 131.445 68.2625) (width 1) (layer B.Cu) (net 11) (status 30))
 (segment (start 132.08 68.2625) (end 131.445 68.2625) (width 1) (layer B.Cu) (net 11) (status 30))
 (segment (start 132.587502 95.059002) (end 132.587502 78.358502) (width 1) (layer B.Cu) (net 11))
 (segment (start 134.4295 96.901) (end 132.587502 95.059002) (width 1) (layer B.Cu) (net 11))
 (segment (start 134.441365 96.912865) (end 134.4295 96.901) (width 1) (layer B.Cu) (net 11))
 (segment (start 133.969 98.044) (end 135.509 98.044) (width 1) (layer F.Cu) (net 11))
 (segment (start 134.4295 96.9645) (end 134.4295 96.901) (width 1) (layer B.Cu) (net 11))
 (segment (start 135.509 98.044) (end 134.4295 96.9645) (width 1) (layer B.Cu) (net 11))
 (via (at 135.509 98.044) (size 0.6) (drill 0.4) (layers F.Cu B.Cu) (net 11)))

